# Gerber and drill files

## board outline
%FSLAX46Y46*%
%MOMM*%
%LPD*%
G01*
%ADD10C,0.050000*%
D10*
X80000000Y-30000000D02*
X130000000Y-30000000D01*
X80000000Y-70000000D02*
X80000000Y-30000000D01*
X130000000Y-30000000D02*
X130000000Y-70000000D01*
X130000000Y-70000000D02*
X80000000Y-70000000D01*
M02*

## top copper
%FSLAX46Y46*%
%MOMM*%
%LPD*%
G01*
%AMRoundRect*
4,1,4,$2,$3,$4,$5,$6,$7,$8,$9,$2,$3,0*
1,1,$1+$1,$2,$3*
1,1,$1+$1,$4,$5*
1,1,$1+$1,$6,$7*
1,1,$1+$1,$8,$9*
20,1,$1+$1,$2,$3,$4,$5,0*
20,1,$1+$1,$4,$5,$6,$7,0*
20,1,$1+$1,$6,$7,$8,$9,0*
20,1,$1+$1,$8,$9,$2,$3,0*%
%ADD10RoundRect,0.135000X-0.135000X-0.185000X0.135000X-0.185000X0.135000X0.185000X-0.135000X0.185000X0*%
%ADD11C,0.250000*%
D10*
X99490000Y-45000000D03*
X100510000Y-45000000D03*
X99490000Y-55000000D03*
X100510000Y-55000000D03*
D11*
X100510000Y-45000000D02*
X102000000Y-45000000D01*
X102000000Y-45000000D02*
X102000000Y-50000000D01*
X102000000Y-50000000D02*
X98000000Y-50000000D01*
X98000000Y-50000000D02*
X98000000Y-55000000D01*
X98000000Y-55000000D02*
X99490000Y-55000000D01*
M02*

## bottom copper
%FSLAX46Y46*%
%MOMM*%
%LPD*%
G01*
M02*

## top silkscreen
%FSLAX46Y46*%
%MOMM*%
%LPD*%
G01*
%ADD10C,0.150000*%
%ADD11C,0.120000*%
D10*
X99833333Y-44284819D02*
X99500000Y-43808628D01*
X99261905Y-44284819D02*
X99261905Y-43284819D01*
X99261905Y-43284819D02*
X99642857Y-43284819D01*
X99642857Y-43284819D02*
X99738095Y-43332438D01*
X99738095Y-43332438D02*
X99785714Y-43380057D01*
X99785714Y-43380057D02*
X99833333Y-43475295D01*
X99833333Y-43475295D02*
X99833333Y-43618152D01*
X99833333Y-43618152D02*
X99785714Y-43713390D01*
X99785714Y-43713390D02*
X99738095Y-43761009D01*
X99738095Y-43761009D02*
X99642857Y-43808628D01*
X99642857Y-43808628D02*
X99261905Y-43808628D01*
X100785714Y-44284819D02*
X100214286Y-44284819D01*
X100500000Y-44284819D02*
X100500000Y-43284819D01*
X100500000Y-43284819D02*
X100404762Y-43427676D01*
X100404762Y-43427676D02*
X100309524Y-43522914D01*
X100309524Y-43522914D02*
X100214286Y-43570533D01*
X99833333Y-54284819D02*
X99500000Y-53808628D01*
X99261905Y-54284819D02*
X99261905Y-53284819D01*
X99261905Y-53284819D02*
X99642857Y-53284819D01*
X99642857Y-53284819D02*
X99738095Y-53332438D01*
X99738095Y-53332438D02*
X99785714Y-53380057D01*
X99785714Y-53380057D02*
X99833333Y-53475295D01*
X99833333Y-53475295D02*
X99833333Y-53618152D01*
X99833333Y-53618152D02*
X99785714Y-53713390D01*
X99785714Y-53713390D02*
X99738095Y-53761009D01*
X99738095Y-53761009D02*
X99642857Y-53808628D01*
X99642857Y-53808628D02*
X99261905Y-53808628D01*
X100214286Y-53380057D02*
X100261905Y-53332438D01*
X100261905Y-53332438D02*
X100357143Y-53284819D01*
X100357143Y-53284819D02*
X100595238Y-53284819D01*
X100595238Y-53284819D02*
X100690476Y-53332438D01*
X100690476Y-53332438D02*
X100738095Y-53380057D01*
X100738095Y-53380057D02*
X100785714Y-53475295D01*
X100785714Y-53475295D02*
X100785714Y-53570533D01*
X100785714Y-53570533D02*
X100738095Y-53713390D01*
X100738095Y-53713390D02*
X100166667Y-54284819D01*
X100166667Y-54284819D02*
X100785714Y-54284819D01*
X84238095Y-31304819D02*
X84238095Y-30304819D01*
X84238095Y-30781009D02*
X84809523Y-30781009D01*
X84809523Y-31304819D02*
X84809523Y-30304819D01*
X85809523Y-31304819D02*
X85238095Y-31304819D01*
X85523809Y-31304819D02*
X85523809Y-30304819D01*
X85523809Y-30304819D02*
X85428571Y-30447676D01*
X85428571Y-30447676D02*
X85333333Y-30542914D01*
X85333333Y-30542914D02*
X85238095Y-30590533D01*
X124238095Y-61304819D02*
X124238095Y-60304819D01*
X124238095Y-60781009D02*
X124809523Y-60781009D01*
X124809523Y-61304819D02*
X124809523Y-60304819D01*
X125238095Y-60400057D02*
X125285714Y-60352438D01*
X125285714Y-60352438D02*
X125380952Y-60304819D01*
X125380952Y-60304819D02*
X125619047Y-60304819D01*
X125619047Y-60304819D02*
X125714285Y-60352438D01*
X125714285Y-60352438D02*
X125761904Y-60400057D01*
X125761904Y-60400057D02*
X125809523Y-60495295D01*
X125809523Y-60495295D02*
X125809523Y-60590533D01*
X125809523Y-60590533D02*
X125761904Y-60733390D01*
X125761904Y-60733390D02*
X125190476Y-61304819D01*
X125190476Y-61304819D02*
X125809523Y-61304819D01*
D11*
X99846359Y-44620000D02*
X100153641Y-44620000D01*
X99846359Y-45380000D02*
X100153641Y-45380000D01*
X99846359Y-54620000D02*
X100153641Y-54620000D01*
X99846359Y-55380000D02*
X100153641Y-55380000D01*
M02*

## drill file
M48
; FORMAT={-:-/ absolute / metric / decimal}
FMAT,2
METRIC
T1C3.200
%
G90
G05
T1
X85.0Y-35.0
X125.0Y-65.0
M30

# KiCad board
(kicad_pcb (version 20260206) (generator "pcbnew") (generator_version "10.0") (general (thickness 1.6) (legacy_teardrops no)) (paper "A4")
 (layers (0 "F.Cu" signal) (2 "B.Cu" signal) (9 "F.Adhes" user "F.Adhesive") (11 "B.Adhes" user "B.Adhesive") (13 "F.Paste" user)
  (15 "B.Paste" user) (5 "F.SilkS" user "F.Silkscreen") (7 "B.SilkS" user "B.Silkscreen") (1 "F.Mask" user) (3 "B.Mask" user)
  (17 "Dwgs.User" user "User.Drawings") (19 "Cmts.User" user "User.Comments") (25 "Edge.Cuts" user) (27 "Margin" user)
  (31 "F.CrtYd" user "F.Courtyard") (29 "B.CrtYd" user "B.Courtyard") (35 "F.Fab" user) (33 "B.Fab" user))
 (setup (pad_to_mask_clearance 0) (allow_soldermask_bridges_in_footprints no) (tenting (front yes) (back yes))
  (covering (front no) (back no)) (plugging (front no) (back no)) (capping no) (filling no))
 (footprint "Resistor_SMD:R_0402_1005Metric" (layer "F.Cu") (at 100 45)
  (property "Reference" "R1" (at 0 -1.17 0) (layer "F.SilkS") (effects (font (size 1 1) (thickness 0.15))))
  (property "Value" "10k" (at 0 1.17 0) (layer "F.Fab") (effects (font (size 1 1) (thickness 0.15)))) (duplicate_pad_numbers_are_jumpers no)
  (fp_line (start -0.153641 -0.38) (end 0.153641 -0.38) (stroke (width 0.12) (type solid)) (layer "F.SilkS"))
  (fp_line (start -0.153641 0.38) (end 0.153641 0.38) (stroke (width 0.12) (type solid)) (layer "F.SilkS"))
  (pad "1" smd roundrect (at -0.51 0) (size 0.54 0.64) (layers "F.Cu" "F.Mask" "F.Paste") (roundrect_rratio 0.25) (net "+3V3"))
  (pad "2" smd roundrect (at 0.51 0) (size 0.54 0.64) (layers "F.Cu" "F.Mask" "F.Paste") (roundrect_rratio 0.25) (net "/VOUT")))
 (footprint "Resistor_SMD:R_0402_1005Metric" (layer "F.Cu") (at 100 55)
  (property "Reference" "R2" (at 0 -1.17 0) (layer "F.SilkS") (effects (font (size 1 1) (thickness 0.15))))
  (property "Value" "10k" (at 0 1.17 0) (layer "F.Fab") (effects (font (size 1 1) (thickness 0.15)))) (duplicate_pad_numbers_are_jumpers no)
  (fp_line (start -0.153641 -0.38) (end 0.153641 -0.38) (stroke (width 0.12) (type solid)) (layer "F.SilkS"))
  (fp_line (start -0.153641 0.38) (end 0.153641 0.38) (stroke (width 0.12) (type solid)) (layer "F.SilkS"))
  (pad "1" smd roundrect (at -0.51 0) (size 0.54 0.64) (layers "F.Cu" "F.Mask" "F.Paste") (roundrect_rratio 0.25) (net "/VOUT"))
  (pad "2" smd roundrect (at 0.51 0) (size 0.54 0.64) (layers "F.Cu" "F.Mask" "F.Paste") (roundrect_rratio 0.25) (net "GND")))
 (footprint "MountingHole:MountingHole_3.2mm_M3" (layer "F.Cu") (at 85 35)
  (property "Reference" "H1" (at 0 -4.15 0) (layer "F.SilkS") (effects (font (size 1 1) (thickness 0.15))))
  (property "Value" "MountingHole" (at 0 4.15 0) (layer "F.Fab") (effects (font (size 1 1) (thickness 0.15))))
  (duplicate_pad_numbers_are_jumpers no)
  (pad "" np_thru_hole circle (at 0 0) (size 3.2 3.2) (drill 3.2) (layers "*.Cu" "*.Mask")))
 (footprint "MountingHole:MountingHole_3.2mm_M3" (layer "F.Cu") (at 125 65)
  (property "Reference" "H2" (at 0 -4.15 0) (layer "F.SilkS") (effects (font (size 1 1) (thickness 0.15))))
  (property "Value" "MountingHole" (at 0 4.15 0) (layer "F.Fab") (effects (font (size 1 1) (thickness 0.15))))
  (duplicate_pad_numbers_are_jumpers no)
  (pad "" np_thru_hole circle (at 0 0) (size 3.2 3.2) (drill 3.2) (layers "*.Cu" "*.Mask")))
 (gr_line (start 80 30) (end 130 30) (stroke (width 0.05) (type default)) (layer "Edge.Cuts"))
 (gr_line (start 80 70) (end 80 30) (stroke (width 0.05) (type default)) (layer "Edge.Cuts"))
 (gr_line (start 130 30) (end 130 70) (stroke (width 0.05) (type default)) (layer "Edge.Cuts"))
 (gr_line (start 130 70) (end 80 70) (stroke (width 0.05) (type default)) (layer "Edge.Cuts"))
 (segment (start 100.51 45) (end 102 45) (width 0.25) (layer "F.Cu") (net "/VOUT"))
 (segment (start 102 45) (end 102 50) (width 0.25) (layer "F.Cu") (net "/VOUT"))
 (segment (start 102 50) (end 98 50) (width 0.25) (layer "F.Cu") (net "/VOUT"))
 (segment (start 98 50) (end 98 55) (width 0.25) (layer "F.Cu") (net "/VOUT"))
 (segment (start 98 55) (end 99.49 55) (width 0.25) (layer "F.Cu") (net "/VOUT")))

